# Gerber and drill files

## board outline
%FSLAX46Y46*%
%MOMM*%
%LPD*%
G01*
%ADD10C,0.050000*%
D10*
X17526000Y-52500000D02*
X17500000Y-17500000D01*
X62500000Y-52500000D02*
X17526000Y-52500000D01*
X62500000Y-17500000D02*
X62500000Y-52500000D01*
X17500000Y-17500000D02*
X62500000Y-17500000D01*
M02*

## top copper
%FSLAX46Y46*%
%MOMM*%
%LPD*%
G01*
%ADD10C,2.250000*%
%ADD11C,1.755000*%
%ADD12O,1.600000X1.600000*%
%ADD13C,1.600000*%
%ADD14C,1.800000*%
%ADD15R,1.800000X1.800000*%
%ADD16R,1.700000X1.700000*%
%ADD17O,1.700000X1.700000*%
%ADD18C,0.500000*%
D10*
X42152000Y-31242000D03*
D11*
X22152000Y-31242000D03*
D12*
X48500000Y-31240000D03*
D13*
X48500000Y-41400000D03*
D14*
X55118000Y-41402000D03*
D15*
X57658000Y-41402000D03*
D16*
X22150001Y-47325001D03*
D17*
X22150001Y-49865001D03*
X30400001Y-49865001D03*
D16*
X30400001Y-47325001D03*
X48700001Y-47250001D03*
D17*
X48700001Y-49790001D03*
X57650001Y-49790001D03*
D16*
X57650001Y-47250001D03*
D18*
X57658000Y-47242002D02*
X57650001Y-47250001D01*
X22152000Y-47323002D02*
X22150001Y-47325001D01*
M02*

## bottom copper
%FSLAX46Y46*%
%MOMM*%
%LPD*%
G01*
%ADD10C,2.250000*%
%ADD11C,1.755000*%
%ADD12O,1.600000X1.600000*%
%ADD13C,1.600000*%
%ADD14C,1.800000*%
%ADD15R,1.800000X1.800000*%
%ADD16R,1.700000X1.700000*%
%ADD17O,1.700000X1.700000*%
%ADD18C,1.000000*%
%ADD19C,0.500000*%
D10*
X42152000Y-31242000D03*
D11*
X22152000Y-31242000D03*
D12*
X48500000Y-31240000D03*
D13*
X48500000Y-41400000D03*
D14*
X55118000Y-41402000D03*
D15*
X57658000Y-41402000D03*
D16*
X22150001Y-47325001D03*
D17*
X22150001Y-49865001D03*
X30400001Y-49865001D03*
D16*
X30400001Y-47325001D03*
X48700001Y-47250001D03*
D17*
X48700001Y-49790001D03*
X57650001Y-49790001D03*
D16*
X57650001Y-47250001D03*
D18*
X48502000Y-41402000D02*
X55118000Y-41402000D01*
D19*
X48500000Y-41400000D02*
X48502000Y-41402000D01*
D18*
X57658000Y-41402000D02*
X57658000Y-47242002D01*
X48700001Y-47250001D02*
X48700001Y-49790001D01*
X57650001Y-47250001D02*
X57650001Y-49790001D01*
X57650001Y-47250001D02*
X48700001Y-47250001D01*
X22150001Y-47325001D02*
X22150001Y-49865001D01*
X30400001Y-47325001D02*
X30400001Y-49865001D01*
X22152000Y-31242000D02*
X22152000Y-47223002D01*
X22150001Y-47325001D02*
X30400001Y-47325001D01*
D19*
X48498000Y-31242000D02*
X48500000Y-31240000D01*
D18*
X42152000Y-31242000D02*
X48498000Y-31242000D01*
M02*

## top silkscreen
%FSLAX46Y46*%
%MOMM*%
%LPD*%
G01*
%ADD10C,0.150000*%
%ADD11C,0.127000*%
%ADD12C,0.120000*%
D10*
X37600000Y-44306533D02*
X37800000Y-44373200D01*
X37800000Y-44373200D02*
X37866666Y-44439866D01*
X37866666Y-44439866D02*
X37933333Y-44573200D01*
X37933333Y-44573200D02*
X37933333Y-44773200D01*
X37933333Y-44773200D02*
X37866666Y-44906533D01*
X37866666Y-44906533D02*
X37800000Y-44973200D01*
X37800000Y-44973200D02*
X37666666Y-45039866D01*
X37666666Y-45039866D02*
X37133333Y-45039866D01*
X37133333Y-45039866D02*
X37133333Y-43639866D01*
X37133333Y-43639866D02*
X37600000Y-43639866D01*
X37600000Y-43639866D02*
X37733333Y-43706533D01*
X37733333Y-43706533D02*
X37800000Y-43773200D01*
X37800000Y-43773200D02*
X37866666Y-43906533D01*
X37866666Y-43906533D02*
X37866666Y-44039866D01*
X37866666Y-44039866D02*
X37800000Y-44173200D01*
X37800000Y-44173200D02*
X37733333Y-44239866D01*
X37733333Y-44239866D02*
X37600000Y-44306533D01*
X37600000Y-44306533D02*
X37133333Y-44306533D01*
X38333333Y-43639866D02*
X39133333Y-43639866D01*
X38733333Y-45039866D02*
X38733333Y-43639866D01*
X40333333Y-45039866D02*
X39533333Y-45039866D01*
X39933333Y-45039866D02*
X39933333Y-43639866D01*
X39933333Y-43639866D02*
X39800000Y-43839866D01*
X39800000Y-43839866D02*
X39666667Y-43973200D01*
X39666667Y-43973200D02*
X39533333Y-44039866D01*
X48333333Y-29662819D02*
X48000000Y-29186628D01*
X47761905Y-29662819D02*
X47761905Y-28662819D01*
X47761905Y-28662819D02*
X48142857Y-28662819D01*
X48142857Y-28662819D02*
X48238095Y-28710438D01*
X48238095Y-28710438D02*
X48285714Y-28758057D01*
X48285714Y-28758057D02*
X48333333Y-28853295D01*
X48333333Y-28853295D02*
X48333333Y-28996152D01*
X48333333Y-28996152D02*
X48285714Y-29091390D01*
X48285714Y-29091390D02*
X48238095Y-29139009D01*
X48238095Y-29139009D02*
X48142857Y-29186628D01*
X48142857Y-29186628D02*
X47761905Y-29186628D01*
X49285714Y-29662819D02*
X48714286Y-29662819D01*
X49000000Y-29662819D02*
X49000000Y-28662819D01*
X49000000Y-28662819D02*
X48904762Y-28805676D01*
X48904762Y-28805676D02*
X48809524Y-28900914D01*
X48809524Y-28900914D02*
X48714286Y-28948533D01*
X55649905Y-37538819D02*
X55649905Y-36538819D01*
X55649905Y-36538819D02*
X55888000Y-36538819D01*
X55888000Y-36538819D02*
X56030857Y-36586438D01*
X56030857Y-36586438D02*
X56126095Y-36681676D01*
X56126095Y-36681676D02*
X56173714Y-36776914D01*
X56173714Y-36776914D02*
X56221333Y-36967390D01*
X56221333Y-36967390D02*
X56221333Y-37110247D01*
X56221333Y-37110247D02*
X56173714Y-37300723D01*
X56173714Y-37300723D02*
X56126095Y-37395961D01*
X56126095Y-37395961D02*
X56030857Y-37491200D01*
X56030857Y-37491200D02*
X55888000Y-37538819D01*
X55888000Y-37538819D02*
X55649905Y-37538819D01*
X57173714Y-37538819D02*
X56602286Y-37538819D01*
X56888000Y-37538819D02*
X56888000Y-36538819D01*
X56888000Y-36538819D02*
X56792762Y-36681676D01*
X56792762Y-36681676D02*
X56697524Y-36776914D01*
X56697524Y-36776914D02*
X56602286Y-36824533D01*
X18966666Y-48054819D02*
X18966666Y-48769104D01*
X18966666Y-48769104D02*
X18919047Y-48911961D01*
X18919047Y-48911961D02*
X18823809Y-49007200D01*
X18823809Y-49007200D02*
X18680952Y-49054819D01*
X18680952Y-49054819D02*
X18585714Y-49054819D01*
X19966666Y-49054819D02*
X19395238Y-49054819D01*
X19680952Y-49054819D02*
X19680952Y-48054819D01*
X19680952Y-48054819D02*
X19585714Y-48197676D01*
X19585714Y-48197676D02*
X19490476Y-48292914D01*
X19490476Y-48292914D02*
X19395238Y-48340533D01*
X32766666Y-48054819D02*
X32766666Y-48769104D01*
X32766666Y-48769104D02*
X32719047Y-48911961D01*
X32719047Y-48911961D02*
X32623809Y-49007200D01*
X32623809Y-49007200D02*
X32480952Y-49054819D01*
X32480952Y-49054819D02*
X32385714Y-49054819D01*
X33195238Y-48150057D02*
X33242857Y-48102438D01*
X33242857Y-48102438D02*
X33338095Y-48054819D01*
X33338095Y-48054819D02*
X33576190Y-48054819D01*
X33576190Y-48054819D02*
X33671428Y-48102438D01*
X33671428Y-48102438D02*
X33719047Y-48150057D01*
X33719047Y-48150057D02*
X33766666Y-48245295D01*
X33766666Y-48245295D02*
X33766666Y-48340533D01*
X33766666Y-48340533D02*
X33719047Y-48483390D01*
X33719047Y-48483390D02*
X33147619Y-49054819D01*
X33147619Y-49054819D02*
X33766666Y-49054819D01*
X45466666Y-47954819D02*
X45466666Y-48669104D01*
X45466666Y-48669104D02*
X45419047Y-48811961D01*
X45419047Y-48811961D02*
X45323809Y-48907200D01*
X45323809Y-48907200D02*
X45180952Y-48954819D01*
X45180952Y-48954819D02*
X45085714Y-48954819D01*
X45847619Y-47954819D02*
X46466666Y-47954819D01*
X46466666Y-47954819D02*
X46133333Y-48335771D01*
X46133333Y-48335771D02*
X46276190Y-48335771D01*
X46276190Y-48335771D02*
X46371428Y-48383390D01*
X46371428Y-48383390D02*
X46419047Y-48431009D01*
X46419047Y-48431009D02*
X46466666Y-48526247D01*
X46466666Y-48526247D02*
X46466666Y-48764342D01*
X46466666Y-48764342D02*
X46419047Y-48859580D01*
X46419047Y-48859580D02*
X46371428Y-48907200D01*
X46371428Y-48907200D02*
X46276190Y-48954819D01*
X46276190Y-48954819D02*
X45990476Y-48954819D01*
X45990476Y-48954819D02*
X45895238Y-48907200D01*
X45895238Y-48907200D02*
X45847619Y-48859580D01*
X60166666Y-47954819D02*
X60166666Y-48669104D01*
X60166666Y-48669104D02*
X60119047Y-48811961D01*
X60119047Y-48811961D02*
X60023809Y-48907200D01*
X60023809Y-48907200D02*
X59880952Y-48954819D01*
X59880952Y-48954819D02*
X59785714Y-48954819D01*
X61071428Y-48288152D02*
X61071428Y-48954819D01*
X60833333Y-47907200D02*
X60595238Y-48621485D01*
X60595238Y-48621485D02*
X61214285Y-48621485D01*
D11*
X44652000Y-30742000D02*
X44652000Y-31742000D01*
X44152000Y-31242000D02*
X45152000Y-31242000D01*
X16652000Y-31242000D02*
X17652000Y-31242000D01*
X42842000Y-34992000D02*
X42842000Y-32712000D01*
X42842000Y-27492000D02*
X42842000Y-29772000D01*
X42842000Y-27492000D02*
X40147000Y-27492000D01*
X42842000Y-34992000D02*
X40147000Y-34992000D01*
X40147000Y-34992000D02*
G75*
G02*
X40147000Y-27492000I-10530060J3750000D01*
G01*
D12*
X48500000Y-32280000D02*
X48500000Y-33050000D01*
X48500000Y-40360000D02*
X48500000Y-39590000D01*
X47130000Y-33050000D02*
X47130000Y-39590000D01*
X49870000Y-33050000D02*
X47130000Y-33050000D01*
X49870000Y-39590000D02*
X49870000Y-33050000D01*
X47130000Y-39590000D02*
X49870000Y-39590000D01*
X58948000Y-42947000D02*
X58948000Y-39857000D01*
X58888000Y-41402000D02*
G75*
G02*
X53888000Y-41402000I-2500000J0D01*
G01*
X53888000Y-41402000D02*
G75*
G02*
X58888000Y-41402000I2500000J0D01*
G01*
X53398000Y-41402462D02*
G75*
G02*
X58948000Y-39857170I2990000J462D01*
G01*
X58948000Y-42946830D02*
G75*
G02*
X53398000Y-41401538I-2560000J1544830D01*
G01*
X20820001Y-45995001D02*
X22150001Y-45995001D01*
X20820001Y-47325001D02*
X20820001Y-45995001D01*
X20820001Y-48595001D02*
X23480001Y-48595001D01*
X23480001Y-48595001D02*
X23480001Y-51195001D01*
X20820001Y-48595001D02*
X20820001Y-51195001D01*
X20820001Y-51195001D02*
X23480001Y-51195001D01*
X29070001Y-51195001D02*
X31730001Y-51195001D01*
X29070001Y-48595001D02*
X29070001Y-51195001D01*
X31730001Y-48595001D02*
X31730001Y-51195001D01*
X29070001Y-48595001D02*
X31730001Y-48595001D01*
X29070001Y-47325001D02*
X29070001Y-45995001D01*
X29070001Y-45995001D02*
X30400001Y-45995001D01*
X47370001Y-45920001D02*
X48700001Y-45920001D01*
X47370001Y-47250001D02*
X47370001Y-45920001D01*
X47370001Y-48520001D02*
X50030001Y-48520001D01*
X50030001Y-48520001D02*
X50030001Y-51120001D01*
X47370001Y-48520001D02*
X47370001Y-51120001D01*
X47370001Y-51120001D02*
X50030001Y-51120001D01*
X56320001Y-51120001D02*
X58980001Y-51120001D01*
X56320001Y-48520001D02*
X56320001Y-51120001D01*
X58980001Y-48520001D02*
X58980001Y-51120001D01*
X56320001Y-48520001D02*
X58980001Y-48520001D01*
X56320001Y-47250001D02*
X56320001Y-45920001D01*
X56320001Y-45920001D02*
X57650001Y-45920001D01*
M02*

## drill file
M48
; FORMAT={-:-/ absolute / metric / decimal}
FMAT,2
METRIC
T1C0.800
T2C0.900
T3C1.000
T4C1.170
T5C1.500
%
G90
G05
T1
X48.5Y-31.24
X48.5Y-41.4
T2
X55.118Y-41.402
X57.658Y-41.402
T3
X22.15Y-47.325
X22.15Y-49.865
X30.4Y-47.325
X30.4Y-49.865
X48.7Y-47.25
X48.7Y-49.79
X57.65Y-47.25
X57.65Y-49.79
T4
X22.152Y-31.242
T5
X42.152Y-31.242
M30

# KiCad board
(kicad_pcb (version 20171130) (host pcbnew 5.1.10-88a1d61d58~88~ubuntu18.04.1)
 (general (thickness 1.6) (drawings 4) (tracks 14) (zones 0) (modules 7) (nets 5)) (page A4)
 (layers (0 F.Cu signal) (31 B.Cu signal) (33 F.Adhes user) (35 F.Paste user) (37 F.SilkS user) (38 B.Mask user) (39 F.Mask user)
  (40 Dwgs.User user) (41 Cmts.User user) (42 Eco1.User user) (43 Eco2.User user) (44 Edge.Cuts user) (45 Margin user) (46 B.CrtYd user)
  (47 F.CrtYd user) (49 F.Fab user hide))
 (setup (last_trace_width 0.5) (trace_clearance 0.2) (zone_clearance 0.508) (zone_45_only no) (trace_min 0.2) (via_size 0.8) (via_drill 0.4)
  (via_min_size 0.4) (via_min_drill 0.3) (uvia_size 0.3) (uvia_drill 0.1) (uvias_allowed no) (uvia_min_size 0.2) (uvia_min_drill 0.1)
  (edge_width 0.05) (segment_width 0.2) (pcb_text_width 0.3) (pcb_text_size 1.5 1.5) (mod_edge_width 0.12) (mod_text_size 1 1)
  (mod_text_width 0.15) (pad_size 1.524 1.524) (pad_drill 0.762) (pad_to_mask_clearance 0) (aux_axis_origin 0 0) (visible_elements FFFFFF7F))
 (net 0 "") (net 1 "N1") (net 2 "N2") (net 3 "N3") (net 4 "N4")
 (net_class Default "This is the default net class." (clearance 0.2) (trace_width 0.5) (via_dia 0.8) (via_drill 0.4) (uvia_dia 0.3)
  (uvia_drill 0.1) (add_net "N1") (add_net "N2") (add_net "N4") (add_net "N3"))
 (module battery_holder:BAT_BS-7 (layer F.Cu) (at 32.152 31.242)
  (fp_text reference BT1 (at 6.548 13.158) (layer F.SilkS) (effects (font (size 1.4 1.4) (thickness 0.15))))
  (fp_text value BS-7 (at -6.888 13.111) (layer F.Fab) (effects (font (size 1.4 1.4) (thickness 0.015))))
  (fp_line (start 12.5 -0.5) (end 12.5 0.5) (layer F.SilkS) (width 0.127))
  (fp_line (start 12 0) (end 13 0) (layer F.SilkS) (width 0.127))
  (fp_line (start -15.5 0) (end -14.5 0) (layer F.SilkS) (width 0.127))
  (fp_line (start 10.69 3.75) (end 10.69 1.47) (layer F.SilkS) (width 0.127))
  (fp_line (start 10.69 -3.75) (end 10.69 -1.47) (layer F.SilkS) (width 0.127))
  (fp_line (start 10.69 -3.75) (end 7.995 -3.75) (layer F.SilkS) (width 0.127))
  (fp_line (start 10.69 3.75) (end 7.995 3.75) (layer F.SilkS) (width 0.127))
  (fp_arc (start -2.53506 0) (end 7.995 3.75) (angle 320.796) (layer F.SilkS) (width 0.127))
  (pad + thru_hole circle (at 10 0) (size 2.25 2.25) (drill 1.5) (layers *.Cu *.Mask) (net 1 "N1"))
  (pad - thru_hole circle (at -10 0) (size 1.755 1.755) (drill 1.17) (layers *.Cu *.Mask) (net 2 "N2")))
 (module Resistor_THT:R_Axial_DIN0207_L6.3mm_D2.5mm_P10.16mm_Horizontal (layer F.Cu) (at 48.5 41.4 90)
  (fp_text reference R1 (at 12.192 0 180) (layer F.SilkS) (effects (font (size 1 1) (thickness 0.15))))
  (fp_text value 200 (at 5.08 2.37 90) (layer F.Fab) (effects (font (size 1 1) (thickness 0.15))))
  (fp_line (start 9.12 0) (end 8.35 0) (layer F.SilkS) (width 0.12))
  (fp_line (start 1.04 0) (end 1.81 0) (layer F.SilkS) (width 0.12))
  (fp_line (start 8.35 -1.37) (end 1.81 -1.37) (layer F.SilkS) (width 0.12))
  (fp_line (start 8.35 1.37) (end 8.35 -1.37) (layer F.SilkS) (width 0.12))
  (fp_line (start 1.81 1.37) (end 8.35 1.37) (layer F.SilkS) (width 0.12))
  (fp_line (start 1.81 -1.37) (end 1.81 1.37) (layer F.SilkS) (width 0.12))
  (pad 2 thru_hole oval (at 10.16 0 90) (size 1.6 1.6) (drill 0.8) (layers *.Cu *.Mask) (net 1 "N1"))
  (pad 1 thru_hole circle (at 0 0 90) (size 1.6 1.6) (drill 0.8) (layers *.Cu *.Mask) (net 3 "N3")))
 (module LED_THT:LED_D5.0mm (layer F.Cu) (at 57.658 41.402 180)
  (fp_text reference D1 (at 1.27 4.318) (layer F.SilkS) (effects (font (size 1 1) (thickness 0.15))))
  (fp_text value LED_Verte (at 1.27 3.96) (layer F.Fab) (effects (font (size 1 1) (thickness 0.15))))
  (fp_line (start -1.29 -1.545) (end -1.29 1.545) (layer F.SilkS) (width 0.12))
  (fp_circle (center 1.27 0) (end 3.77 0) (layer F.SilkS) (width 0.12))
  (fp_arc (start 1.27 0) (end -1.29 1.54483) (angle -148.9) (layer F.SilkS) (width 0.12))
  (fp_arc (start 1.27 0) (end -1.29 -1.54483) (angle 148.9) (layer F.SilkS) (width 0.12))
  (pad 2 thru_hole circle (at 2.54 0 180) (size 1.8 1.8) (drill 0.9) (layers *.Cu *.Mask) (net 3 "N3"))
  (pad 1 thru_hole rect (at 0 0 180) (size 1.8 1.8) (drill 0.9) (layers *.Cu *.Mask) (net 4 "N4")))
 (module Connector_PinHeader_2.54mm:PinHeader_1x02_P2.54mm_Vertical (layer F.Cu) (at 22.150001 47.325001)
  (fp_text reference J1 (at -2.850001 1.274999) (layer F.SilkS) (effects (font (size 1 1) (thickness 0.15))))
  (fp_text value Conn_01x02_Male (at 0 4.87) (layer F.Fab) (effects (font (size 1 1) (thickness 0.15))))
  (fp_line (start -1.33 -1.33) (end 0 -1.33) (layer F.SilkS) (width 0.12))
  (fp_line (start -1.33 0) (end -1.33 -1.33) (layer F.SilkS) (width 0.12))
  (fp_line (start -1.33 1.27) (end 1.33 1.27) (layer F.SilkS) (width 0.12))
  (fp_line (start 1.33 1.27) (end 1.33 3.87) (layer F.SilkS) (width 0.12))
  (fp_line (start -1.33 1.27) (end -1.33 3.87) (layer F.SilkS) (width 0.12))
  (fp_line (start -1.33 3.87) (end 1.33 3.87) (layer F.SilkS) (width 0.12))
  (pad 1 thru_hole rect (at 0 0) (size 1.7 1.7) (drill 1) (layers *.Cu *.Mask) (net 2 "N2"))
  (pad 2 thru_hole oval (at 0 2.54) (size 1.7 1.7) (drill 1) (layers *.Cu *.Mask) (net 2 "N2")))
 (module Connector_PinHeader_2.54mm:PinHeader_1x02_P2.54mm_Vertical (layer F.Cu) (at 30.400001 47.325001)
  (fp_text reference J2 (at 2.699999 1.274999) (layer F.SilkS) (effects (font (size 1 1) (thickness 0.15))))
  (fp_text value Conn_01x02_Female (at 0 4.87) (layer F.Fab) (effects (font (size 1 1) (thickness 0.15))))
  (fp_line (start -1.33 3.87) (end 1.33 3.87) (layer F.SilkS) (width 0.12))
  (fp_line (start -1.33 1.27) (end -1.33 3.87) (layer F.SilkS) (width 0.12))
  (fp_line (start 1.33 1.27) (end 1.33 3.87) (layer F.SilkS) (width 0.12))
  (fp_line (start -1.33 1.27) (end 1.33 1.27) (layer F.SilkS) (width 0.12))
  (fp_line (start -1.33 0) (end -1.33 -1.33) (layer F.SilkS) (width 0.12))
  (fp_line (start -1.33 -1.33) (end 0 -1.33) (layer F.SilkS) (width 0.12))
  (pad 2 thru_hole oval (at 0 2.54) (size 1.7 1.7) (drill 1) (layers *.Cu *.Mask) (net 2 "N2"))
  (pad 1 thru_hole rect (at 0 0) (size 1.7 1.7) (drill 1) (layers *.Cu *.Mask) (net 2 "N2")))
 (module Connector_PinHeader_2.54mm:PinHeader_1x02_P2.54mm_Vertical (layer F.Cu) (at 48.700001 47.250001)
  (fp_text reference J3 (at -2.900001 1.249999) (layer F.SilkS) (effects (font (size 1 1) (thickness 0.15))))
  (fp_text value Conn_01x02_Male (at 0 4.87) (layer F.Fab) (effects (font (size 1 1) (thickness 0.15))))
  (fp_line (start -1.33 -1.33) (end 0 -1.33) (layer F.SilkS) (width 0.12))
  (fp_line (start -1.33 0) (end -1.33 -1.33) (layer F.SilkS) (width 0.12))
  (fp_line (start -1.33 1.27) (end 1.33 1.27) (layer F.SilkS) (width 0.12))
  (fp_line (start 1.33 1.27) (end 1.33 3.87) (layer F.SilkS) (width 0.12))
  (fp_line (start -1.33 1.27) (end -1.33 3.87) (layer F.SilkS) (width 0.12))
  (fp_line (start -1.33 3.87) (end 1.33 3.87) (layer F.SilkS) (width 0.12))
  (pad 1 thru_hole rect (at 0 0) (size 1.7 1.7) (drill 1) (layers *.Cu *.Mask) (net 4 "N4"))
  (pad 2 thru_hole oval (at 0 2.54) (size 1.7 1.7) (drill 1) (layers *.Cu *.Mask) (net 4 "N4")))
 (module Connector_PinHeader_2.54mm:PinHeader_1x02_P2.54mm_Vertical (layer F.Cu) (at 57.650001 47.250001)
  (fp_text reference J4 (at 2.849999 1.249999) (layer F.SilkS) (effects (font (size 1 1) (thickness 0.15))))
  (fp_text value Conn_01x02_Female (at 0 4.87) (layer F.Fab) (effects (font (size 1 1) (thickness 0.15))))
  (fp_line (start -1.33 3.87) (end 1.33 3.87) (layer F.SilkS) (width 0.12))
  (fp_line (start -1.33 1.27) (end -1.33 3.87) (layer F.SilkS) (width 0.12))
  (fp_line (start 1.33 1.27) (end 1.33 3.87) (layer F.SilkS) (width 0.12))
  (fp_line (start -1.33 1.27) (end 1.33 1.27) (layer F.SilkS) (width 0.12))
  (fp_line (start -1.33 0) (end -1.33 -1.33) (layer F.SilkS) (width 0.12))
  (fp_line (start -1.33 -1.33) (end 0 -1.33) (layer F.SilkS) (width 0.12))
  (pad 2 thru_hole oval (at 0 2.54) (size 1.7 1.7) (drill 1) (layers *.Cu *.Mask) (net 4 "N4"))
  (pad 1 thru_hole rect (at 0 0) (size 1.7 1.7) (drill 1) (layers *.Cu *.Mask) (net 4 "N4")))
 (gr_line (start 17.526 52.5) (end 17.5 17.5) (layer Edge.Cuts) (width 0.05))
 (gr_line (start 62.5 52.5) (end 17.526 52.5) (layer Edge.Cuts) (width 0.05))
 (gr_line (start 62.5 17.5) (end 62.5 52.5) (layer Edge.Cuts) (width 0.05))
 (gr_line (start 17.5 17.5) (end 62.5 17.5) (layer Edge.Cuts) (width 0.05))
 (segment (start 48.502 41.402) (end 55.118 41.402) (width 1) (layer B.Cu) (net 3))
 (segment (start 48.5 41.4) (end 48.502 41.402) (width 0.5) (layer B.Cu) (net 3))
 (segment (start 57.658 47.242002) (end 57.650001 47.250001) (width 0.5) (layer F.Cu) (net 4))
 (segment (start 57.658 41.402) (end 57.658 47.242002) (width 1) (layer B.Cu) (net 4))
 (segment (start 48.700001 47.250001) (end 48.700001 49.790001) (width 1) (layer B.Cu) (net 4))
 (segment (start 57.650001 47.250001) (end 57.650001 49.790001) (width 1) (layer B.Cu) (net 4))
 (segment (start 57.650001 47.250001) (end 48.700001 47.250001) (width 1) (layer B.Cu) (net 4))
 (segment (start 22.152 47.323002) (end 22.150001 47.325001) (width 0.5) (layer F.Cu) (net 2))
 (segment (start 22.150001 47.325001) (end 22.150001 49.865001) (width 1) (layer B.Cu) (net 2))
 (segment (start 30.400001 47.325001) (end 30.400001 49.865001) (width 1) (layer B.Cu) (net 2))
 (segment (start 22.152 31.242) (end 22.152 47.223002) (width 1) (layer B.Cu) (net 2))
 (segment (start 22.150001 47.325001) (end 30.400001 47.325001) (width 1) (layer B.Cu) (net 2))
 (segment (start 48.498 31.242) (end 48.5 31.24) (width 0.5) (layer B.Cu) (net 1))
 (segment (start 42.152 31.242) (end 48.498 31.242) (width 1) (layer B.Cu) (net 1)))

